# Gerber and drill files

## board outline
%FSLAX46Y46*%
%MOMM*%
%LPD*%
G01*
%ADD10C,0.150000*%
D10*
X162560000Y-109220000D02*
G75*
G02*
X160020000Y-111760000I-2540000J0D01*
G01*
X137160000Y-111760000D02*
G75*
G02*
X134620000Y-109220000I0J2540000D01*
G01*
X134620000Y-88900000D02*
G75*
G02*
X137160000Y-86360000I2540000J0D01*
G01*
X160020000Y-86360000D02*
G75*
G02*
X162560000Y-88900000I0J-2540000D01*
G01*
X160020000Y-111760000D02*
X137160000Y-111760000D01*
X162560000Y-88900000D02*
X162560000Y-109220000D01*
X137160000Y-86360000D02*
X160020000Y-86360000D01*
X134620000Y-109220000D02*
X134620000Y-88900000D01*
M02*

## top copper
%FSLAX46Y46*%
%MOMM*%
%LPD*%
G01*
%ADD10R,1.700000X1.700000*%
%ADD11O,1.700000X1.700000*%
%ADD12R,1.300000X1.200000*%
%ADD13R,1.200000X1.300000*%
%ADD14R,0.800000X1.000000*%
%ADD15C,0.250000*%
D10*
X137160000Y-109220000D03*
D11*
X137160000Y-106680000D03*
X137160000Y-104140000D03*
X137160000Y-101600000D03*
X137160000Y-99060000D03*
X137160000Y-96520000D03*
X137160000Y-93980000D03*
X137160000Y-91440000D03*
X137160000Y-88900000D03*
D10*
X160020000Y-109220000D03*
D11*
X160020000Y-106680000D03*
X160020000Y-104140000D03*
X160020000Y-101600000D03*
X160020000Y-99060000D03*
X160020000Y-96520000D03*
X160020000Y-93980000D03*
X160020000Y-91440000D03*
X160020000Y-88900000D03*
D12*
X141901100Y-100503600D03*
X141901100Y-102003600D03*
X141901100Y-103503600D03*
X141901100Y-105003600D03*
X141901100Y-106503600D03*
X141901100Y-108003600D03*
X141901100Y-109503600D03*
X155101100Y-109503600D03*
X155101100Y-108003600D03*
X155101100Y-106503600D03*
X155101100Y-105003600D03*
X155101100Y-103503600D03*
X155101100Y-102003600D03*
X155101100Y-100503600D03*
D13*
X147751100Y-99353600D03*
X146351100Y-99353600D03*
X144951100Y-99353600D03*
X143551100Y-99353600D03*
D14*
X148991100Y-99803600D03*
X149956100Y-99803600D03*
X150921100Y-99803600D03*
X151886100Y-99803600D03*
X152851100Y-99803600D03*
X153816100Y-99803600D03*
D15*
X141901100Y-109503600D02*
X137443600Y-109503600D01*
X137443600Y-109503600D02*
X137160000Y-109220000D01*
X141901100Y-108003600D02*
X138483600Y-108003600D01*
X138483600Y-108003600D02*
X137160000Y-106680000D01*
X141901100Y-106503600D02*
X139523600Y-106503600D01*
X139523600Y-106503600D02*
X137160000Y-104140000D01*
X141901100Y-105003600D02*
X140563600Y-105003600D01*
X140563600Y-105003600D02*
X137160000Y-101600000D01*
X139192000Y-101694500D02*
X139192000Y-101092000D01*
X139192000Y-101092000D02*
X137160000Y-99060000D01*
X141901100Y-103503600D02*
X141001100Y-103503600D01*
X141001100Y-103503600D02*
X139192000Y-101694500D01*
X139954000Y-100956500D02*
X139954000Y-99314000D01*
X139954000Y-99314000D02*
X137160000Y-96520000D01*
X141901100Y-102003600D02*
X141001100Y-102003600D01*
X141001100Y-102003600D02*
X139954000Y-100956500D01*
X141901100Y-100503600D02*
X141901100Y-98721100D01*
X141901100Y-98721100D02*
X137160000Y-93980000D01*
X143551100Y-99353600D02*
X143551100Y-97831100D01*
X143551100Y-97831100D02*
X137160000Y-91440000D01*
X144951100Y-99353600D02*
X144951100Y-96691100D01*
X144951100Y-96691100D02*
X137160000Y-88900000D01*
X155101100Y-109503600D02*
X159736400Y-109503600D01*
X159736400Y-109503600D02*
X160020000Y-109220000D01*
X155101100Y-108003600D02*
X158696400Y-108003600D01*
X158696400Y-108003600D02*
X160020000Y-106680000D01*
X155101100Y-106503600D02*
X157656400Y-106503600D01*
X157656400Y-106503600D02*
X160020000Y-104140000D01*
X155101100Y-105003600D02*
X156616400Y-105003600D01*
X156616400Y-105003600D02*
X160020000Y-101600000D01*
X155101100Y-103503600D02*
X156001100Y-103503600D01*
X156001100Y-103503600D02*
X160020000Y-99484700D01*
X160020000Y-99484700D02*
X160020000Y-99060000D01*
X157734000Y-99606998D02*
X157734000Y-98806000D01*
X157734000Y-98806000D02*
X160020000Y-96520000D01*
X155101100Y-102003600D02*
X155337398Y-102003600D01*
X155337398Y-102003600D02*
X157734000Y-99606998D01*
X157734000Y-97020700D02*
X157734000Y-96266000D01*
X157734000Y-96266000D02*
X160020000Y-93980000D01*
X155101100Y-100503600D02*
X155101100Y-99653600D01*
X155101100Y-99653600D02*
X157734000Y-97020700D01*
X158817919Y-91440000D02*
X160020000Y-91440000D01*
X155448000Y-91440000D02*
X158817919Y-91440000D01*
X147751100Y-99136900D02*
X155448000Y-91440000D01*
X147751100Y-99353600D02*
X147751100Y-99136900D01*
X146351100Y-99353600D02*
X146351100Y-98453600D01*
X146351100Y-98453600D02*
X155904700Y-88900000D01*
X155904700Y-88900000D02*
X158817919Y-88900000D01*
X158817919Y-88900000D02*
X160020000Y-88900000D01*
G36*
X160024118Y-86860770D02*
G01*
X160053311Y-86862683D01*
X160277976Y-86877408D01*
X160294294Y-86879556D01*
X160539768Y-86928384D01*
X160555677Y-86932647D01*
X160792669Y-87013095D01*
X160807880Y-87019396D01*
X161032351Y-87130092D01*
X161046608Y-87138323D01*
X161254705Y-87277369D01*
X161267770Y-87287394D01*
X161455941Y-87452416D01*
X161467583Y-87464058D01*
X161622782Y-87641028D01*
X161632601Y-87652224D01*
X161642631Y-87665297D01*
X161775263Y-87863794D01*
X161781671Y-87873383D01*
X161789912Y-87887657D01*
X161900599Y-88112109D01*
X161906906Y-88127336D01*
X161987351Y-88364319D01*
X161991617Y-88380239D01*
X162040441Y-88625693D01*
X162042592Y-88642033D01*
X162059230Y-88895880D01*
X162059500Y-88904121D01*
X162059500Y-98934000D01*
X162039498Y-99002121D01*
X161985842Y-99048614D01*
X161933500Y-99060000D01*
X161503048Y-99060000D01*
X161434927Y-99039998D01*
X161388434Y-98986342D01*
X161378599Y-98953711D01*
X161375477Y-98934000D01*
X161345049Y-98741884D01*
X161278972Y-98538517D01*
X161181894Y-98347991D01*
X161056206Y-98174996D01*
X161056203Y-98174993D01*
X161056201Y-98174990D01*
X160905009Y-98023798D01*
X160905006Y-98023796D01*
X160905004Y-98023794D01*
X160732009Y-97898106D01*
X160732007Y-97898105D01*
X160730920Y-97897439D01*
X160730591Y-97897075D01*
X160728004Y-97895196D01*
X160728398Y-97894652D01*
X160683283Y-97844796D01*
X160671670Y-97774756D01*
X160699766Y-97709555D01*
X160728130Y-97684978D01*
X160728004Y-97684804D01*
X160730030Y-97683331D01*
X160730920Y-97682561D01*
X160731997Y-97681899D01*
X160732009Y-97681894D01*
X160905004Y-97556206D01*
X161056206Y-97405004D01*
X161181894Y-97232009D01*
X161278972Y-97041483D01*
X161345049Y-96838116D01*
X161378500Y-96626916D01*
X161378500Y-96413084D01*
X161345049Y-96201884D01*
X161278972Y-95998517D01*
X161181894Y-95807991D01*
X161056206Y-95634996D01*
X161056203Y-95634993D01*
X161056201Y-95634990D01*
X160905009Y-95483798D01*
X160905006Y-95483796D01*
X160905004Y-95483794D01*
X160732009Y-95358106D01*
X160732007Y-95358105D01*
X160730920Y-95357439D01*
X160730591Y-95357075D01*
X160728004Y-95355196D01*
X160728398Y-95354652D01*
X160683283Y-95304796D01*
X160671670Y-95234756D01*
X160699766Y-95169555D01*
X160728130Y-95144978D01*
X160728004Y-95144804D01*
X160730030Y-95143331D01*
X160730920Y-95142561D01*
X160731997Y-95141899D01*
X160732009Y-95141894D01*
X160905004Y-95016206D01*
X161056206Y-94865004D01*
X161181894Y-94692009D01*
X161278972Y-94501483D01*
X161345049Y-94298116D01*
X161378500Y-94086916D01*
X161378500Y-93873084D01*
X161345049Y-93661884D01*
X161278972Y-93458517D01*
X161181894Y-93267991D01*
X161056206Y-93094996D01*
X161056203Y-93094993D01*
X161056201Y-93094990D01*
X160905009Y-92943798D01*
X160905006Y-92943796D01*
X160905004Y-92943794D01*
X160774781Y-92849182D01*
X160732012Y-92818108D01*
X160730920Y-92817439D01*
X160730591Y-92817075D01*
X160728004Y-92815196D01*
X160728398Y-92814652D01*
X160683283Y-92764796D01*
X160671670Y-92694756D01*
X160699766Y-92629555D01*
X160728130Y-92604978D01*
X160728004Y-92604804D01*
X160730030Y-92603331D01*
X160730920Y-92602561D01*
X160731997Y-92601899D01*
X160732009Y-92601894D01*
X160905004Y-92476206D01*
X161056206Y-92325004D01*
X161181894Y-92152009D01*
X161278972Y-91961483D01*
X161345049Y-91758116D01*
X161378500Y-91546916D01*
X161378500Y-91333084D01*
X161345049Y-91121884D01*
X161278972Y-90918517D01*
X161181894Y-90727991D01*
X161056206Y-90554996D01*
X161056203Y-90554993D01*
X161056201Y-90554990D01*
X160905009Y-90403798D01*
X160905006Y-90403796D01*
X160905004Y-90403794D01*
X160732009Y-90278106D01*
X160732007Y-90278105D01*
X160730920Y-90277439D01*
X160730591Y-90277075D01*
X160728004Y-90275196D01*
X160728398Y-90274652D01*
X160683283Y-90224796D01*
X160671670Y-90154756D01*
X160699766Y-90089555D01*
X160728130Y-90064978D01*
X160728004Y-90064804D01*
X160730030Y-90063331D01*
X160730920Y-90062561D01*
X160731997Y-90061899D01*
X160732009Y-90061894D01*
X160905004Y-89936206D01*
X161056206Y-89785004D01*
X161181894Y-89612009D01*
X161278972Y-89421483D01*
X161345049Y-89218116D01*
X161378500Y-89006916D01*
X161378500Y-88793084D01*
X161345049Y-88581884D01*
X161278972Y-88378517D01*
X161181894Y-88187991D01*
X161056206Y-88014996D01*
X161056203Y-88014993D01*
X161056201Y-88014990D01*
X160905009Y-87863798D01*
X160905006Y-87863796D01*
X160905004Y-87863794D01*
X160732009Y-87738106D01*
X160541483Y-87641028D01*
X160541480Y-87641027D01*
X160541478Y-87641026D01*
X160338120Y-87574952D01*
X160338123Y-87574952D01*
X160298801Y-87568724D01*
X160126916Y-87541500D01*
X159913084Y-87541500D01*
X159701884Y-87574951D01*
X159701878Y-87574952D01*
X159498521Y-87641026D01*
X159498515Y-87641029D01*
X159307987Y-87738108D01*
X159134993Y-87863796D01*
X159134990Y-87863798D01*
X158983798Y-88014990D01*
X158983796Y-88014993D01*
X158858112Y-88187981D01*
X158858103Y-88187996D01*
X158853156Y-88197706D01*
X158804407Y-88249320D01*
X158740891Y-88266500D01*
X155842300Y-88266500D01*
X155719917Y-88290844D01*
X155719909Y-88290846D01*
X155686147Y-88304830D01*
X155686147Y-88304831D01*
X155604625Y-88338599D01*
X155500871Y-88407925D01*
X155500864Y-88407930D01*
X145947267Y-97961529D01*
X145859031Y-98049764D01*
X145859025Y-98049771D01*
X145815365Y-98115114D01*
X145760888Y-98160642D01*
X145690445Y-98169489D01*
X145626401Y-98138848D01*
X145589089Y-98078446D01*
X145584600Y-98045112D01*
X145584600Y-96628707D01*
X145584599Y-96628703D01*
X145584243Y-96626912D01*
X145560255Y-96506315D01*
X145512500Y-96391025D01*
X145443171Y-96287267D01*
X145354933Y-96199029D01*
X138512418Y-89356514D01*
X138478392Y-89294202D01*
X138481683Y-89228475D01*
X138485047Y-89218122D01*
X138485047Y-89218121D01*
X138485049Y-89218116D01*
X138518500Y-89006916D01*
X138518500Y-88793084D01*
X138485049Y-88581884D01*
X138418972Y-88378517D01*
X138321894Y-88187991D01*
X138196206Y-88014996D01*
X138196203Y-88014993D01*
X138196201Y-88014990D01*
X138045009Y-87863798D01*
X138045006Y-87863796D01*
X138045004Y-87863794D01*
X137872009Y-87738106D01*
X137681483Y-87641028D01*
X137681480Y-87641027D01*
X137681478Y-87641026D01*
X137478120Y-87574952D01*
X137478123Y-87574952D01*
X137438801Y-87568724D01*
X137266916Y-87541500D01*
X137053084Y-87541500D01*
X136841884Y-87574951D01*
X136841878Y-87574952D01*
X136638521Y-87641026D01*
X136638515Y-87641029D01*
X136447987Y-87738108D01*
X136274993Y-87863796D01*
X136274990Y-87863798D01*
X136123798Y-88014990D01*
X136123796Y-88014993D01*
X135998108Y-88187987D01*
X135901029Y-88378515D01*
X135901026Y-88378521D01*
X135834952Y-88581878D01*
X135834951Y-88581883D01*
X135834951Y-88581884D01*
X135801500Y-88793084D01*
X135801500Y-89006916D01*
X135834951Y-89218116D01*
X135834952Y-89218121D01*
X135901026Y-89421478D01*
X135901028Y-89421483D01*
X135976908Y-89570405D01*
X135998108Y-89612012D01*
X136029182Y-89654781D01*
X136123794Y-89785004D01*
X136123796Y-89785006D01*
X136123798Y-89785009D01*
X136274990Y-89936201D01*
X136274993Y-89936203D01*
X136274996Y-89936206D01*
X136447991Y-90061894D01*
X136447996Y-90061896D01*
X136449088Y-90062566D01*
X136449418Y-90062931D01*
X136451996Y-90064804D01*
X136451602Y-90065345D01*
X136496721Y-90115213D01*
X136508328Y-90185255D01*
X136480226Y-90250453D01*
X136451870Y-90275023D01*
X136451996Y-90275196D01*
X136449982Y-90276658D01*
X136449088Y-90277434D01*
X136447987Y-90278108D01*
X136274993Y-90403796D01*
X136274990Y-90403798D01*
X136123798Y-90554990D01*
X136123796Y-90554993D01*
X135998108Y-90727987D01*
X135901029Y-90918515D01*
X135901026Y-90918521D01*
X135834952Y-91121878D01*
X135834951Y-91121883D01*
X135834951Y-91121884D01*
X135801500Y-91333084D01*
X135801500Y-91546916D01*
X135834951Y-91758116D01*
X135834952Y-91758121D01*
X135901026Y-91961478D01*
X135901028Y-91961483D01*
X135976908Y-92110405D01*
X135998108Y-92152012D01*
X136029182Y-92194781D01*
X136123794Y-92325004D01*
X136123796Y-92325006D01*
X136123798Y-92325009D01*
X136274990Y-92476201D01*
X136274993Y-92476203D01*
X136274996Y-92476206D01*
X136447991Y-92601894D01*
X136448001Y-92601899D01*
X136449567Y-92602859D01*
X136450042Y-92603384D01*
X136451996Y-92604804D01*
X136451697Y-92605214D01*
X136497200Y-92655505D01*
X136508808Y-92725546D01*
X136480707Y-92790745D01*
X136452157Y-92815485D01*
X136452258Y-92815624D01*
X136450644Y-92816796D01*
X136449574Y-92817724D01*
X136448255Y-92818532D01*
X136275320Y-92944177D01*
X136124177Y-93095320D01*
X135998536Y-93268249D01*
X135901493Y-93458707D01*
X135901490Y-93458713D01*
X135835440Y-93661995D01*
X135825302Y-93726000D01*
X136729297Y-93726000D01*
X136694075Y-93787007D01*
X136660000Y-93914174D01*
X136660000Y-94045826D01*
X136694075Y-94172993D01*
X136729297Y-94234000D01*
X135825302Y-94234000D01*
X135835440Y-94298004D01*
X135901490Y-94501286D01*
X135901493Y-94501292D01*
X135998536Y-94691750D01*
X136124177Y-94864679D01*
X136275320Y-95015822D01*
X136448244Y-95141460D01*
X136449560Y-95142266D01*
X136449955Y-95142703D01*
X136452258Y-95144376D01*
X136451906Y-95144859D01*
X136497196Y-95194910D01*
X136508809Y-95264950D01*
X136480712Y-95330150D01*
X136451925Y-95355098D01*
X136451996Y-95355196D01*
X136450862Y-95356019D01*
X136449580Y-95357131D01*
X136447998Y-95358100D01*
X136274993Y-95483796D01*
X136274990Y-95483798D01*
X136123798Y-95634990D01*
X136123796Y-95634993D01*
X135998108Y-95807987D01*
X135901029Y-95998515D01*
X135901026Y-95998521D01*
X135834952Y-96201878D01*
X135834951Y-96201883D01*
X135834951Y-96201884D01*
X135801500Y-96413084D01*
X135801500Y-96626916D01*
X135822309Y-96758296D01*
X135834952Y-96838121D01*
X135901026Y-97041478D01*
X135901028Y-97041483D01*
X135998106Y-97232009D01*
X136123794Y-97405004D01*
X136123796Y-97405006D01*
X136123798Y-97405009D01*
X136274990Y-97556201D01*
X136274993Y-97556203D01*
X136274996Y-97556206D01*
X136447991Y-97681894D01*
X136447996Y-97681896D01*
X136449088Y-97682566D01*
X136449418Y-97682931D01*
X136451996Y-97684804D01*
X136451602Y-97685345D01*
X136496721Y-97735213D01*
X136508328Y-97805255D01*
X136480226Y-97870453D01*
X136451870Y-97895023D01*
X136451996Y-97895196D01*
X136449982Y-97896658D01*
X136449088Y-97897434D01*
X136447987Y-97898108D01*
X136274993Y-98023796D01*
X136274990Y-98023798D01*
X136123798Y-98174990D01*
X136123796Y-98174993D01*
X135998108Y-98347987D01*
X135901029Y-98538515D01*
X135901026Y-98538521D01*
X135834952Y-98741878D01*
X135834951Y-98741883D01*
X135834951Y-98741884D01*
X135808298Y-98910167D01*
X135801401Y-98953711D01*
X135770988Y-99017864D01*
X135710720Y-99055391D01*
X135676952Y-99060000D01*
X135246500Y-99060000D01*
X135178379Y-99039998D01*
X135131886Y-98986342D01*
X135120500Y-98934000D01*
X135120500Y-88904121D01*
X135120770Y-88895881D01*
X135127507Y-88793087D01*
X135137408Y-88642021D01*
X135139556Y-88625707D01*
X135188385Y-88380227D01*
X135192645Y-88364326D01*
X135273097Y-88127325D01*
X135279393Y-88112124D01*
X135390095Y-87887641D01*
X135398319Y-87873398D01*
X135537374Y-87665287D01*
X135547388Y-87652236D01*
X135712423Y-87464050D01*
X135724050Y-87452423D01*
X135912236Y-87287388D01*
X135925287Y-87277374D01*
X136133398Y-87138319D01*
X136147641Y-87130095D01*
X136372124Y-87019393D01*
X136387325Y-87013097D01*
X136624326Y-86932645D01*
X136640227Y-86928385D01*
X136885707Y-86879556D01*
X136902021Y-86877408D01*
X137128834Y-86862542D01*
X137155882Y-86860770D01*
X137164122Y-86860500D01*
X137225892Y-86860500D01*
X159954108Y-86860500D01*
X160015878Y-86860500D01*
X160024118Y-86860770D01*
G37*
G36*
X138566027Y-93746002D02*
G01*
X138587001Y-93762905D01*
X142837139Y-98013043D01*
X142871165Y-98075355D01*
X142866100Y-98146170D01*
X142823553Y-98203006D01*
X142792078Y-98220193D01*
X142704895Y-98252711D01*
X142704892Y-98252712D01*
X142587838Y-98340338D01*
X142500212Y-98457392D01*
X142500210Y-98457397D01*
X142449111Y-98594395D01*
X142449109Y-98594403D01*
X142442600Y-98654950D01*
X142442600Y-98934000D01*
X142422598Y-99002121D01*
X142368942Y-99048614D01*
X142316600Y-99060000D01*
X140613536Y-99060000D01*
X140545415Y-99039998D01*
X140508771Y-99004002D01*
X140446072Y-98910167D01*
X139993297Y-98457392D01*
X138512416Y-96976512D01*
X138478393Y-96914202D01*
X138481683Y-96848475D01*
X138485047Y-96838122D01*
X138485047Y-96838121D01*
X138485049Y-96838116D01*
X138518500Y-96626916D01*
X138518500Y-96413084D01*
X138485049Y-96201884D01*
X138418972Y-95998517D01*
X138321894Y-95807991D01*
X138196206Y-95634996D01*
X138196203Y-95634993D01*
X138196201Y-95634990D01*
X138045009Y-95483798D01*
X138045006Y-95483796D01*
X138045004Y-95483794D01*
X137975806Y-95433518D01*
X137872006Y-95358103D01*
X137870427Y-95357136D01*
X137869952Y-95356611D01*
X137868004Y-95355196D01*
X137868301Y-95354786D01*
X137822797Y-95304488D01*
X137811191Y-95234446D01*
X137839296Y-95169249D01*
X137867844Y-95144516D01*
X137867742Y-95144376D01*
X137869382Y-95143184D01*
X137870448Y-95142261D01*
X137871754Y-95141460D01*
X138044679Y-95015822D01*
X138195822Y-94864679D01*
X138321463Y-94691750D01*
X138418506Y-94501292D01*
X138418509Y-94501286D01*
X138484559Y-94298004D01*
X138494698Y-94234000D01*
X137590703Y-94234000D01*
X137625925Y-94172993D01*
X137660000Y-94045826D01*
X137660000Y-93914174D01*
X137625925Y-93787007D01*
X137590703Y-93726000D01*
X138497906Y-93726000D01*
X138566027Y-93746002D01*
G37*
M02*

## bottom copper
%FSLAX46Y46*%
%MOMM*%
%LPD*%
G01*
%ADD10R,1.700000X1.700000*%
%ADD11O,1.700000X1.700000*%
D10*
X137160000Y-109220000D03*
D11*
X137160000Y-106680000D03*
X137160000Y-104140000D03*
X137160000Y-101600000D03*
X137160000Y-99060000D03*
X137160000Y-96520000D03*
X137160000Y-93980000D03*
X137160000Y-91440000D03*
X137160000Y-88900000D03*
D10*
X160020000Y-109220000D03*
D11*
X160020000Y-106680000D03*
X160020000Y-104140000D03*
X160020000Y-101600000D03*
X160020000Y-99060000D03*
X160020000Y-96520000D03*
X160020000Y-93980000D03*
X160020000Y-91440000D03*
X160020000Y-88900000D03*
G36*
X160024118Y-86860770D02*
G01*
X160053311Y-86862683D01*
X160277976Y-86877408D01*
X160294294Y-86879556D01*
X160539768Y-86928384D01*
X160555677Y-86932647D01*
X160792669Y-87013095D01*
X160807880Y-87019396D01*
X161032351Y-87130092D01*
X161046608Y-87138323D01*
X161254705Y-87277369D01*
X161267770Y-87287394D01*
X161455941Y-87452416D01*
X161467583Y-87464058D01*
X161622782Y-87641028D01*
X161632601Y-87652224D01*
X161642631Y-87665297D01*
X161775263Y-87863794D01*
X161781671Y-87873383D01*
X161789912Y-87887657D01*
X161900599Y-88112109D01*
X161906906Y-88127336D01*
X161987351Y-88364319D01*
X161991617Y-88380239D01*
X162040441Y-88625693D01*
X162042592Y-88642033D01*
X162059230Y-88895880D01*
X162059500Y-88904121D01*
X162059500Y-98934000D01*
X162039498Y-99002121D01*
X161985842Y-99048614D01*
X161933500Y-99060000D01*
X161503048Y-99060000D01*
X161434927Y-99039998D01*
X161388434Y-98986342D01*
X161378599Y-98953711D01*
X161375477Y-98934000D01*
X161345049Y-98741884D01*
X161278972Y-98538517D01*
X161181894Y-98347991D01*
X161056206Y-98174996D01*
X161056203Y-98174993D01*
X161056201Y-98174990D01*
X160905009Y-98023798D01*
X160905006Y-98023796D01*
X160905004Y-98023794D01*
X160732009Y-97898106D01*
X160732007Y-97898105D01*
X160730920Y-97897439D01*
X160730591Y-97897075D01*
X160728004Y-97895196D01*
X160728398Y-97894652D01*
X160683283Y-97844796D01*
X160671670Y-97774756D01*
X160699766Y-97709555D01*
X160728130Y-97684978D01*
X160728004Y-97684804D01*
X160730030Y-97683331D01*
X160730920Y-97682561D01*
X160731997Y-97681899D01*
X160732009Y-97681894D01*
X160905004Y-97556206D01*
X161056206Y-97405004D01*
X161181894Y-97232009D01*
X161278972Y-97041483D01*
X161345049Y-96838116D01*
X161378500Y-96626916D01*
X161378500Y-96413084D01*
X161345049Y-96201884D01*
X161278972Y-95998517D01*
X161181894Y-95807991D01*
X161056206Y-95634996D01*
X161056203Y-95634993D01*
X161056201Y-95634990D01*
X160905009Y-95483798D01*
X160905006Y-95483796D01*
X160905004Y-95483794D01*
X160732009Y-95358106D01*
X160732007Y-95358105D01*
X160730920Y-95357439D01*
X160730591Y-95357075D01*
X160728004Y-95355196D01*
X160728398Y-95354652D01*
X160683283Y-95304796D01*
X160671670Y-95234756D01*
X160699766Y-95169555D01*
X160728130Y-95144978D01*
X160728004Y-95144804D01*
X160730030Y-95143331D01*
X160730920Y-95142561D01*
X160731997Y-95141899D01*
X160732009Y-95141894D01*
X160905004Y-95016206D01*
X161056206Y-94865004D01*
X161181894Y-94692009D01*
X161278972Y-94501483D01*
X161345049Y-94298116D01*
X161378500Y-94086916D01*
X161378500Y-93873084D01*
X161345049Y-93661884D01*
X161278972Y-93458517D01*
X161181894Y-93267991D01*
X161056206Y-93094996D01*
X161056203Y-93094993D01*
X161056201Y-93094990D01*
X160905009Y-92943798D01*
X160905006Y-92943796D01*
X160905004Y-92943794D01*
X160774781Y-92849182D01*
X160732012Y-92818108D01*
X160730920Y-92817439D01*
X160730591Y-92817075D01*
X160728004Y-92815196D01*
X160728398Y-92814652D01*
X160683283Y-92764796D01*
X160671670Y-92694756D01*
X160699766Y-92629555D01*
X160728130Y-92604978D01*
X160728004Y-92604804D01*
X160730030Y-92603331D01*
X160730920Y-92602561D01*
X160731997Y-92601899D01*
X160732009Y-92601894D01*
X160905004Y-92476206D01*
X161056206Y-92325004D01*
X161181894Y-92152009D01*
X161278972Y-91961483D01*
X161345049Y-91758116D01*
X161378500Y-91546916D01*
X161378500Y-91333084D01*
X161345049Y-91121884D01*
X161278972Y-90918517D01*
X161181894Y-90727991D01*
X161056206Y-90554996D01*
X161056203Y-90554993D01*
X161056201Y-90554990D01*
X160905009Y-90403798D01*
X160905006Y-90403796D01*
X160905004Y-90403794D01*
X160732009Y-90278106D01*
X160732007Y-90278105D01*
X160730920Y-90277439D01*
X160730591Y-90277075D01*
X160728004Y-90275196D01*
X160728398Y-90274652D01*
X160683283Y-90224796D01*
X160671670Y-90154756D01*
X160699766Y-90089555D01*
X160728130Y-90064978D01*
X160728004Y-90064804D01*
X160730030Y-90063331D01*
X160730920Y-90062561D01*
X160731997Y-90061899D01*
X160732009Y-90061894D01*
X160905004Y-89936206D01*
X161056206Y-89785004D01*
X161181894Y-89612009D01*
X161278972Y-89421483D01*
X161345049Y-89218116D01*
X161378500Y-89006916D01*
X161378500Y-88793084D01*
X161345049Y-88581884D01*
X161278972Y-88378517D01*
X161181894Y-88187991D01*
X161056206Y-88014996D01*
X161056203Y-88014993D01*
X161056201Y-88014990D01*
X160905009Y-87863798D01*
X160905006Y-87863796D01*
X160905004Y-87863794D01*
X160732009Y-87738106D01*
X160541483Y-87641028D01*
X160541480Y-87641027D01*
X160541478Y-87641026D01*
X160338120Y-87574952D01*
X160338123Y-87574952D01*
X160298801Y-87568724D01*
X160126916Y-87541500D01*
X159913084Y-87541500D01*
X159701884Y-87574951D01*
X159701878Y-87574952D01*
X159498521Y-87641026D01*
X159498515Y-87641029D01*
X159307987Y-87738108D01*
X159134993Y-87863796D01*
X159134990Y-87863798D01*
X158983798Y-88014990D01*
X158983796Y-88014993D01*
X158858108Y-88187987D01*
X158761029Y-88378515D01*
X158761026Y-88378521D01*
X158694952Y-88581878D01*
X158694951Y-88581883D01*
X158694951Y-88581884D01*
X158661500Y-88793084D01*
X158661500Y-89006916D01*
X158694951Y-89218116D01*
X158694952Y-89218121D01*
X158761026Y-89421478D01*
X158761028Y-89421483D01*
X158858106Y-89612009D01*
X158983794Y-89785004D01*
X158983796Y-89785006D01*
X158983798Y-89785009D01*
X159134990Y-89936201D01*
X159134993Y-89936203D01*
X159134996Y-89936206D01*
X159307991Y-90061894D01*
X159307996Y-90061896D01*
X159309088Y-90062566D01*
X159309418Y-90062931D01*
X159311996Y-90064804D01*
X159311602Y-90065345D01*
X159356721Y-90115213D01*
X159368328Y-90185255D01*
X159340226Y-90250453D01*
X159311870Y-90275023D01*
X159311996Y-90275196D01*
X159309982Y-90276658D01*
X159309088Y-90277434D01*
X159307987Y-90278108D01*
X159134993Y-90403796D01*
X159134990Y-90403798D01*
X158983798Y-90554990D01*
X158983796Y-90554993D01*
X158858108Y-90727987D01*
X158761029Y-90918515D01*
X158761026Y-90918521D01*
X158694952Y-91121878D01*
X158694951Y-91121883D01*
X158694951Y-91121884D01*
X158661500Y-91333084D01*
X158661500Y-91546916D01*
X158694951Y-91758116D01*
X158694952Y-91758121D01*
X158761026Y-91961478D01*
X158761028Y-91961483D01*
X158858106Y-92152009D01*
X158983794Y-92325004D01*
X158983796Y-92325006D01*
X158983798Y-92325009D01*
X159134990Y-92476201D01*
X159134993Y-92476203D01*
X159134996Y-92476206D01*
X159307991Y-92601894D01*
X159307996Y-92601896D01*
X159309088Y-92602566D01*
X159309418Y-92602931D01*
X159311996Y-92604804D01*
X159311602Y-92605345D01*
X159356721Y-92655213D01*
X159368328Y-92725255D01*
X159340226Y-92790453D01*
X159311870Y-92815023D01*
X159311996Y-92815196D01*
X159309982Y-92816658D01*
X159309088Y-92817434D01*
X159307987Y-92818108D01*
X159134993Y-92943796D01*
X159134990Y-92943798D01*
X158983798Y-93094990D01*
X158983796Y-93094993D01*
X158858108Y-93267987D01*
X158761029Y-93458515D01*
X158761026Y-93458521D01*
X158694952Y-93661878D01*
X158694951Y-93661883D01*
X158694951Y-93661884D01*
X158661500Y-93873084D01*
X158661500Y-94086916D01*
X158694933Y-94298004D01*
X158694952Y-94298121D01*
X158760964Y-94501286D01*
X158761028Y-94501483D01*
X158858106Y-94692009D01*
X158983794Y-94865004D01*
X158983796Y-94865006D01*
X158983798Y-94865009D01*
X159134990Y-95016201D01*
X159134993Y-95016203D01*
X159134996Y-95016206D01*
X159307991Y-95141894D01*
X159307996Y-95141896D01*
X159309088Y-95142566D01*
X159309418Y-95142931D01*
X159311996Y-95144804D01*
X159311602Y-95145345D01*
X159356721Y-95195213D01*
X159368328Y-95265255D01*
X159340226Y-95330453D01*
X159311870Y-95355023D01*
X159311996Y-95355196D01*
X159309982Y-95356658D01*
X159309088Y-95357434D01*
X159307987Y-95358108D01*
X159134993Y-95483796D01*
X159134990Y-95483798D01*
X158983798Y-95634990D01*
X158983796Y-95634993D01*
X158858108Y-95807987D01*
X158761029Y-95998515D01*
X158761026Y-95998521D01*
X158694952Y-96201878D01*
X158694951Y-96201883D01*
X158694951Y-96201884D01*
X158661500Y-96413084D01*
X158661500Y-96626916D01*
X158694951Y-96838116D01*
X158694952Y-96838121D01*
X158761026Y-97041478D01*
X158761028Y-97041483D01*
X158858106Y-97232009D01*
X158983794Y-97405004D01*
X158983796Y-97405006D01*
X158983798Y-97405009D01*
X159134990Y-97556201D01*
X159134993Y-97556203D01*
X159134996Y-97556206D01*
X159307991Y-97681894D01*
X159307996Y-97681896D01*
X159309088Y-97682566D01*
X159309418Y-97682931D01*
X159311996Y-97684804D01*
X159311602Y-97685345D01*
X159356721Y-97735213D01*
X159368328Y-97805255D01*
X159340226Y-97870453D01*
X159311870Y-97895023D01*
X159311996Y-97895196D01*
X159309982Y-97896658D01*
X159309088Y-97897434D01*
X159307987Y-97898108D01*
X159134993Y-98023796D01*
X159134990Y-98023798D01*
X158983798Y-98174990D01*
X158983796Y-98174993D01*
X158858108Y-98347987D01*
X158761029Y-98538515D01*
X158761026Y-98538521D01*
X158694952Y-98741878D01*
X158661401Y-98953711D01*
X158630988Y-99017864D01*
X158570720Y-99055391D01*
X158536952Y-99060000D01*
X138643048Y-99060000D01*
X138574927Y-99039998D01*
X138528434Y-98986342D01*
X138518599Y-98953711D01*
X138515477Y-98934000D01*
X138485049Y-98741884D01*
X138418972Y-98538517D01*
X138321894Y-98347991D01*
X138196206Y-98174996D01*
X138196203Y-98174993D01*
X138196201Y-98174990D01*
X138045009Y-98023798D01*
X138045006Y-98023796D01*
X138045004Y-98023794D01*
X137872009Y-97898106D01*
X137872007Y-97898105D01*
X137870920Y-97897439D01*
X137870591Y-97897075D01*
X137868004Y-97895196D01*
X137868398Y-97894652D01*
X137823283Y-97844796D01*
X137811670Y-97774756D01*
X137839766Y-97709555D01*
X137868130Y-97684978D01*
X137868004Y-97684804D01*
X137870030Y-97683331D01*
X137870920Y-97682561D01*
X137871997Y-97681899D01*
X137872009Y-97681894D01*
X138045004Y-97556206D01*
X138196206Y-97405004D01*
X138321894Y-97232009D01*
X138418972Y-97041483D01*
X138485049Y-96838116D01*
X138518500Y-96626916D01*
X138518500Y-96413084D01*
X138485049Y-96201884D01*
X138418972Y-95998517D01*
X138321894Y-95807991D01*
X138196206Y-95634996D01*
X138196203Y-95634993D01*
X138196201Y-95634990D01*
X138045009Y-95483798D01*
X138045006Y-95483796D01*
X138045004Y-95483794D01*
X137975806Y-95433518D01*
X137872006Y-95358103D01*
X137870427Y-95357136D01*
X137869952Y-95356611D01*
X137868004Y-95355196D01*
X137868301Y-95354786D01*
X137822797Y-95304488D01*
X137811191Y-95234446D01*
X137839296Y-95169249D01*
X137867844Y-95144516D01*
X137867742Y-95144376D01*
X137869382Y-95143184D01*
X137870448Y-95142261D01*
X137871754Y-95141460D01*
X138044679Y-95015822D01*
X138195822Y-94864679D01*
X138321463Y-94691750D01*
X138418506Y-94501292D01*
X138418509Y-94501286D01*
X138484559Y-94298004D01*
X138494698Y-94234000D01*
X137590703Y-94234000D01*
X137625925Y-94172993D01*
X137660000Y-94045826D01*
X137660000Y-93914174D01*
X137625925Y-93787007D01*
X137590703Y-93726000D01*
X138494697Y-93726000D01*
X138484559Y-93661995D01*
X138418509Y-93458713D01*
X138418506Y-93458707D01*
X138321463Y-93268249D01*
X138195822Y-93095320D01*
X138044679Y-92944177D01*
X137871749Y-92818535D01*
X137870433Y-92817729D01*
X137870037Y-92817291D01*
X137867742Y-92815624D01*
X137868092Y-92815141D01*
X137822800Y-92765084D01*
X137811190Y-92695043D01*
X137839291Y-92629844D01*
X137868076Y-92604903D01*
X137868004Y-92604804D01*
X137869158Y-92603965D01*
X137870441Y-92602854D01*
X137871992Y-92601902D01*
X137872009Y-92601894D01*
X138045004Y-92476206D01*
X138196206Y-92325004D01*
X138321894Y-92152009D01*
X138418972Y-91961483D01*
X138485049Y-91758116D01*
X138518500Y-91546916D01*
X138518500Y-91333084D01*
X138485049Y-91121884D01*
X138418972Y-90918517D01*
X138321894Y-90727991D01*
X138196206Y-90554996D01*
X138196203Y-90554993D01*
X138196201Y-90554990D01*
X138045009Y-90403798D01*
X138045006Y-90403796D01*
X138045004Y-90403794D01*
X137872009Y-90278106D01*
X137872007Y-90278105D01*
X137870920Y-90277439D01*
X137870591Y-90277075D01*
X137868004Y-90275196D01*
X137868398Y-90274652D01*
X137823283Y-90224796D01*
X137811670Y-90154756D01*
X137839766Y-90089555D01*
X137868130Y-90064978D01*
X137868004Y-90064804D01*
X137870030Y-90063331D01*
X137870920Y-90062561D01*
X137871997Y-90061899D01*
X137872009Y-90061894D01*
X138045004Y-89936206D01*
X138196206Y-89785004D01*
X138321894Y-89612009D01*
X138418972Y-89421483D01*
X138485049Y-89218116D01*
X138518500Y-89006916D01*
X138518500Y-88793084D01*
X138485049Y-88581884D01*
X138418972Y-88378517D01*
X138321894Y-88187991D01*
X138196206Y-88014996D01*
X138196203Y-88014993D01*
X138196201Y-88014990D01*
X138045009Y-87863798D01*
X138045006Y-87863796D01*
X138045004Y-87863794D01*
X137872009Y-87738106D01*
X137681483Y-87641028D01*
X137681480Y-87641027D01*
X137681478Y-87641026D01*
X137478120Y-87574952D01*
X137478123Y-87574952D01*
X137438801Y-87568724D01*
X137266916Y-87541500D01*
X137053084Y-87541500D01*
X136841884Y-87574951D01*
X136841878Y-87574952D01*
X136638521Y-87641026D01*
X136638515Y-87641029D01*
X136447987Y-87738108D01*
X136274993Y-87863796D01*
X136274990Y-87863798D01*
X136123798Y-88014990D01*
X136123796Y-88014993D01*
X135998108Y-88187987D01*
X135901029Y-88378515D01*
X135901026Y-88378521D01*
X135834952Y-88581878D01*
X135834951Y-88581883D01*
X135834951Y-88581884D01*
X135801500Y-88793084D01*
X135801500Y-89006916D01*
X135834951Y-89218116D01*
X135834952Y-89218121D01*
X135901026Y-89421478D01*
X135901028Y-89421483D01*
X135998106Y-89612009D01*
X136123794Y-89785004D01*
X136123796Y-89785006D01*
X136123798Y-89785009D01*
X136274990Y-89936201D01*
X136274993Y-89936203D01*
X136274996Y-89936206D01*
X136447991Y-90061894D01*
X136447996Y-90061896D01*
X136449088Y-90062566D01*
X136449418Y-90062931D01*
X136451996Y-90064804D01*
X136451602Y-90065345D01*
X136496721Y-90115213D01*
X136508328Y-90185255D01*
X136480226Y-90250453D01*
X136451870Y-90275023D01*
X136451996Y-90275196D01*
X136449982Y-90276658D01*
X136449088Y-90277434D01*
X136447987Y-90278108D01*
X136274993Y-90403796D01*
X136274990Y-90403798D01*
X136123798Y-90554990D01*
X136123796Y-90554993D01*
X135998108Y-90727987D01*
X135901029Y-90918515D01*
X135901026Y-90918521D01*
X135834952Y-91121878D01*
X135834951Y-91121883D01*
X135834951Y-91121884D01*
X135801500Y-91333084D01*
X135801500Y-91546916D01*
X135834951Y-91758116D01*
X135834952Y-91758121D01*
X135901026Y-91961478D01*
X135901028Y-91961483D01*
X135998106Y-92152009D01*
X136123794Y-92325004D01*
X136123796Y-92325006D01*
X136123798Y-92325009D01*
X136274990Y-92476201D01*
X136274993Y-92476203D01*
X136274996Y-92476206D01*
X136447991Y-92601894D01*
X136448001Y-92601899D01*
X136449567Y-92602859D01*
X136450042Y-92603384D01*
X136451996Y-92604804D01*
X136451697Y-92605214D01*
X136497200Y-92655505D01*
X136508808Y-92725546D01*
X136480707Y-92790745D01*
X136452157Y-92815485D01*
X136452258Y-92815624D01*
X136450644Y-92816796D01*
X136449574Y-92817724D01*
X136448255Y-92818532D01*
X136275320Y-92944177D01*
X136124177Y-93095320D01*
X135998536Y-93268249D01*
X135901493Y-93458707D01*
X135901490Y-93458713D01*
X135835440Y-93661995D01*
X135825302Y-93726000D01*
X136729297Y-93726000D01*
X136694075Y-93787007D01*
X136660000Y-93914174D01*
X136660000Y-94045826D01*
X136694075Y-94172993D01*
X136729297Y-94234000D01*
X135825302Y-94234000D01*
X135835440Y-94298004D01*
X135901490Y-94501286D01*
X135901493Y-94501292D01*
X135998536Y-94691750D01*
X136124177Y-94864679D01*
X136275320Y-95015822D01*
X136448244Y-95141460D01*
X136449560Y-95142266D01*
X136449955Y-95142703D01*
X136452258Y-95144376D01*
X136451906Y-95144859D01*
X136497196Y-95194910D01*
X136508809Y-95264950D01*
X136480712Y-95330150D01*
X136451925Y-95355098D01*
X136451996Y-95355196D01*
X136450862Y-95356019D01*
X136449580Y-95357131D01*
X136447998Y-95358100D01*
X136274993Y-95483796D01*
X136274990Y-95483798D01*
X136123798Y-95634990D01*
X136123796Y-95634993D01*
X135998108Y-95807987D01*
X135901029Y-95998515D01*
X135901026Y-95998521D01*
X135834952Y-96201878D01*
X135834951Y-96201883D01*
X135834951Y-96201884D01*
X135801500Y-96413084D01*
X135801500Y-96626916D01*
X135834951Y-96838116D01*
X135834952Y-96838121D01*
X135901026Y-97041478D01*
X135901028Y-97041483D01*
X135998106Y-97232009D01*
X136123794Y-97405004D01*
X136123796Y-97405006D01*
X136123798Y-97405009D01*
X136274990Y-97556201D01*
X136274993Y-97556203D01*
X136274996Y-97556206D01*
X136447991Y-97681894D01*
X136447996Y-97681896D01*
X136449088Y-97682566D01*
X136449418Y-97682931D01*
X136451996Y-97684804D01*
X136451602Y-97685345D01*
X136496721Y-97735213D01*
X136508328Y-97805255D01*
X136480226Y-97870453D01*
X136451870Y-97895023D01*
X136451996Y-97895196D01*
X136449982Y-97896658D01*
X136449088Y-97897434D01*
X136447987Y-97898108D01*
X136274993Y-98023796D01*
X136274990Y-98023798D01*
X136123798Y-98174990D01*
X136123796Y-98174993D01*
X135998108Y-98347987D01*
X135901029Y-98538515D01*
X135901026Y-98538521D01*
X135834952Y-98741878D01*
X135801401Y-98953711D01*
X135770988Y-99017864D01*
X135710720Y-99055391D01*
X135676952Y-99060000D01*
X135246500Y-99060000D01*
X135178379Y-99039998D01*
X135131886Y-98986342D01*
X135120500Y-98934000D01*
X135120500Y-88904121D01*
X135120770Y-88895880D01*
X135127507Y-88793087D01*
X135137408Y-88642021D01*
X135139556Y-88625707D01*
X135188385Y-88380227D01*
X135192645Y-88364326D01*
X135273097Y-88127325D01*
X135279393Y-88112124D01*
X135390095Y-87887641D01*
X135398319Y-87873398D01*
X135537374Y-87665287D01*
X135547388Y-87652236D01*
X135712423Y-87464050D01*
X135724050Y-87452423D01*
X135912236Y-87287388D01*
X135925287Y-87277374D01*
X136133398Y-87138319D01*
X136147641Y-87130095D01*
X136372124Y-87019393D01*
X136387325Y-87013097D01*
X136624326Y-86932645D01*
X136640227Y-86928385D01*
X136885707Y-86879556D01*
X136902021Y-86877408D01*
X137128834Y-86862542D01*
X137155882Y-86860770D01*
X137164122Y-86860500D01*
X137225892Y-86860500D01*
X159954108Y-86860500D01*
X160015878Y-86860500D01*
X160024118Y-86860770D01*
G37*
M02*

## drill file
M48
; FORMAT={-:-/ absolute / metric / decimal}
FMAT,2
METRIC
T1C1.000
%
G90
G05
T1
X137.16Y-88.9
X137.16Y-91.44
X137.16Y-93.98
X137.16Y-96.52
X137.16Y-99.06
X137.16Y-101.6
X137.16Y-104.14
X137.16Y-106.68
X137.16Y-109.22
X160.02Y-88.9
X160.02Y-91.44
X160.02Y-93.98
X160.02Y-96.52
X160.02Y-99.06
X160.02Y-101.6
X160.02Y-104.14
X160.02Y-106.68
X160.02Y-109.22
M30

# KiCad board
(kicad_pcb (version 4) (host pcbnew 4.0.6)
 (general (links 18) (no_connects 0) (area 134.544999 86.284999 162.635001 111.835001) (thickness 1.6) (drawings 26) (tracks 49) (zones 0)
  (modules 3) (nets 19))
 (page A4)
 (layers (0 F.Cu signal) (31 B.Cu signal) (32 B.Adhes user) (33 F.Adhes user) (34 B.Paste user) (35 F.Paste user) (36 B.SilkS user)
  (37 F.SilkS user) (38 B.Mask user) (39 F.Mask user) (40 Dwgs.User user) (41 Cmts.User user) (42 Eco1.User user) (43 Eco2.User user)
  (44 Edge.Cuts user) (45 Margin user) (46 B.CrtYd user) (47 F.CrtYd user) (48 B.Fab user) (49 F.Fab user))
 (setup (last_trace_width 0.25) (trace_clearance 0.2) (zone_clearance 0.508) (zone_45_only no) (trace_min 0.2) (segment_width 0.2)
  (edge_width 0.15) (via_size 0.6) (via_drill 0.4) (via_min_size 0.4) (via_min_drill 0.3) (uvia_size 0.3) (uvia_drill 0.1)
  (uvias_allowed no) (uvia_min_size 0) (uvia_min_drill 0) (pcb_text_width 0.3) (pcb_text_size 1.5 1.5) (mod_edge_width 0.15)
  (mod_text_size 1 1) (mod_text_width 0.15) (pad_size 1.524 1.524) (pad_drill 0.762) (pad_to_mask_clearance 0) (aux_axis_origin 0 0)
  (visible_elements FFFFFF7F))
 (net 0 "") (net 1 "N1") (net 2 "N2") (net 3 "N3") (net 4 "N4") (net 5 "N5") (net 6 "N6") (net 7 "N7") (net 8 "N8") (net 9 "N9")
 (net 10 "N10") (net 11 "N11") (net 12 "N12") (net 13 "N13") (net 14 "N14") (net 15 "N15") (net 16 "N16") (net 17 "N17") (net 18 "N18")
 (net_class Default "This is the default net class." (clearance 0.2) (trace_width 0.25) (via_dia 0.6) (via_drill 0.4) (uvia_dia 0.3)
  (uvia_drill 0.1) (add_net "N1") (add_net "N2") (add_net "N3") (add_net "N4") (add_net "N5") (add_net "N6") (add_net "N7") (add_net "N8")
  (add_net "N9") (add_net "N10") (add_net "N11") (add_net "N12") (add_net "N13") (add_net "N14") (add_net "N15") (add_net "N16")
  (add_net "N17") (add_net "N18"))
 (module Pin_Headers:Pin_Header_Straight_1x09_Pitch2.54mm (layer F.Cu) (at 137.16 109.22 180)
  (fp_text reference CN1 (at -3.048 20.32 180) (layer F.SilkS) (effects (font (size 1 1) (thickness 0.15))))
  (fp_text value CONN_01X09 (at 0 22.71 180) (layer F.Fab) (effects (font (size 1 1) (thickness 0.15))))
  (pad 1 thru_hole rect (at 0 0 180) (size 1.7 1.7) (drill 1) (layers *.Cu *.Mask) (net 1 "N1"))
  (pad 2 thru_hole oval (at 0 2.54 180) (size 1.7 1.7) (drill 1) (layers *.Cu *.Mask) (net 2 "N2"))
  (pad 3 thru_hole oval (at 0 5.08 180) (size 1.7 1.7) (drill 1) (layers *.Cu *.Mask) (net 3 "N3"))
  (pad 4 thru_hole oval (at 0 7.62 180) (size 1.7 1.7) (drill 1) (layers *.Cu *.Mask) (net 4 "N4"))
  (pad 5 thru_hole oval (at 0 10.16 180) (size 1.7 1.7) (drill 1) (layers *.Cu *.Mask) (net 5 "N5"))
  (pad 6 thru_hole oval (at 0 12.7 180) (size 1.7 1.7) (drill 1) (layers *.Cu *.Mask) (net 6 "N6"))
  (pad 7 thru_hole oval (at 0 15.24 180) (size 1.7 1.7) (drill 1) (layers *.Cu *.Mask) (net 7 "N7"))
  (pad 8 thru_hole oval (at 0 17.78 180) (size 1.7 1.7) (drill 1) (layers *.Cu *.Mask) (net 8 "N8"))
  (pad 9 thru_hole oval (at 0 20.32 180) (size 1.7 1.7) (drill 1) (layers *.Cu *.Mask) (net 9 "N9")))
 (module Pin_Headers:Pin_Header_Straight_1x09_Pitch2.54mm (layer F.Cu) (at 160.02 109.22 180)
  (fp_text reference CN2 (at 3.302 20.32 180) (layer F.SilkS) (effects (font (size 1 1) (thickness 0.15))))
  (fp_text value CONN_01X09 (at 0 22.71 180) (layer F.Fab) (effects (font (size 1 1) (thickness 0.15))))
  (pad 1 thru_hole rect (at 0 0 180) (size 1.7 1.7) (drill 1) (layers *.Cu *.Mask) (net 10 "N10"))
  (pad 2 thru_hole oval (at 0 2.54 180) (size 1.7 1.7) (drill 1) (layers *.Cu *.Mask) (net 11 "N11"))
  (pad 3 thru_hole oval (at 0 5.08 180) (size 1.7 1.7) (drill 1) (layers *.Cu *.Mask) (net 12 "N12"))
  (pad 4 thru_hole oval (at 0 7.62 180) (size 1.7 1.7) (drill 1) (layers *.Cu *.Mask) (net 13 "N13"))
  (pad 5 thru_hole oval (at 0 10.16 180) (size 1.7 1.7) (drill 1) (layers *.Cu *.Mask) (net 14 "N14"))
  (pad 6 thru_hole oval (at 0 12.7 180) (size 1.7 1.7) (drill 1) (layers *.Cu *.Mask) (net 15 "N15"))
  (pad 7 thru_hole oval (at 0 15.24 180) (size 1.7 1.7) (drill 1) (layers *.Cu *.Mask) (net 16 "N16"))
  (pad 8 thru_hole oval (at 0 17.78 180) (size 1.7 1.7) (drill 1) (layers *.Cu *.Mask) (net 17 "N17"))
  (pad 9 thru_hole oval (at 0 20.32 180) (size 1.7 1.7) (drill 1) (layers *.Cu *.Mask) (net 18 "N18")))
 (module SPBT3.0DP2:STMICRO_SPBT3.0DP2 (layer F.Cu) (at 148.5011 105.0036)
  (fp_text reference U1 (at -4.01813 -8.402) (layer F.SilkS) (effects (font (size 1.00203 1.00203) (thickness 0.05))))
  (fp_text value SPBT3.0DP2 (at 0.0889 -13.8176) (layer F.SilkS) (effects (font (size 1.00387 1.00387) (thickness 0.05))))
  (pad 1 smd rect (at -6.6 -4.5 270) (size 1.2 1.3) (layers F.Cu F.Paste F.Mask) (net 7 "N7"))
  (pad 2 smd rect (at -6.6 -3 270) (size 1.2 1.3) (layers F.Cu F.Paste F.Mask) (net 6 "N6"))
  (pad 3 smd rect (at -6.6 -1.5 270) (size 1.2 1.3) (layers F.Cu F.Paste F.Mask) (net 5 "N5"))
  (pad 4 smd rect (at -6.6 0 270) (size 1.2 1.3) (layers F.Cu F.Paste F.Mask) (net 4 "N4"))
  (pad 5 smd rect (at -6.6 1.5 270) (size 1.2 1.3) (layers F.Cu F.Paste F.Mask) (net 3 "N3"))
  (pad 6 smd rect (at -6.6 3 270) (size 1.2 1.3) (layers F.Cu F.Paste F.Mask) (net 2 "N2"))
  (pad 7 smd rect (at -6.6 4.5 270) (size 1.2 1.3) (layers F.Cu F.Paste F.Mask) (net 1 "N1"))
  (pad 8 smd rect (at 6.6 4.5 270) (size 1.2 1.3) (layers F.Cu F.Paste F.Mask) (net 10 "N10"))
  (pad 9 smd rect (at 6.6 3 270) (size 1.2 1.3) (layers F.Cu F.Paste F.Mask) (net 11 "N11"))
  (pad 10 smd rect (at 6.6 1.5 270) (size 1.2 1.3) (layers F.Cu F.Paste F.Mask) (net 12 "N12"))
  (pad 11 smd rect (at 6.6 0 270) (size 1.2 1.3) (layers F.Cu F.Paste F.Mask) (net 13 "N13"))
  (pad 12 smd rect (at 6.6 -1.5 270) (size 1.2 1.3) (layers F.Cu F.Paste F.Mask) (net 14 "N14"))
  (pad 13 smd rect (at 6.6 -3 270) (size 1.2 1.3) (layers F.Cu F.Paste F.Mask) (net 15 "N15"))
  (pad 14 smd rect (at 6.6 -4.5 270) (size 1.2 1.3) (layers F.Cu F.Paste F.Mask) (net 16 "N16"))
  (pad 15 smd rect (at -0.75 -5.65) (size 1.2 1.3) (layers F.Cu F.Paste F.Mask) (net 17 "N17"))
  (pad 16 smd rect (at -2.15 -5.65) (size 1.2 1.3) (layers F.Cu F.Paste F.Mask) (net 18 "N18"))
  (pad 17 smd rect (at -3.55 -5.65) (size 1.2 1.3) (layers F.Cu F.Paste F.Mask) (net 9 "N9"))
  (pad 18 smd rect (at -4.95 -5.65) (size 1.2 1.3) (layers F.Cu F.Paste F.Mask) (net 8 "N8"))
  (pad P$6 smd rect (at 0.49 -5.2) (size 0.8 1) (layers F.Cu F.Paste F.Mask))
  (pad P$5 smd rect (at 1.455 -5.2) (size 0.8 1) (layers F.Cu F.Paste F.Mask))
  (pad P$4 smd rect (at 2.42 -5.2) (size 0.8 1) (layers F.Cu F.Paste F.Mask))
  (pad P$3 smd rect (at 3.385 -5.2) (size 0.8 1) (layers F.Cu F.Paste F.Mask))
  (pad P$2 smd rect (at 4.35 -5.2) (size 0.8 1) (layers F.Cu F.Paste F.Mask))
  (pad P$1 smd rect (at 5.315 -5.2) (size 0.8 1) (layers F.Cu F.Paste F.Mask)))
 (gr_arc (start 160.02 109.22) (end 162.56 109.22) (angle 90) (layer Edge.Cuts) (width 0.15))
 (gr_arc (start 137.16 109.22) (end 137.16 111.76) (angle 90) (layer Edge.Cuts) (width 0.15))
 (gr_arc (start 137.16 88.9) (end 134.62 88.9) (angle 90) (layer Edge.Cuts) (width 0.15))
 (gr_arc (start 160.02 88.9) (end 160.02 86.36) (angle 90) (layer Edge.Cuts) (width 0.15))
 (gr_line (start 160.02 111.76) (end 137.16 111.76) (layer Edge.Cuts) (width 0.15))
 (gr_line (start 162.56 88.9) (end 162.56 109.22) (layer Edge.Cuts) (width 0.15))
 (gr_line (start 137.16 86.36) (end 160.02 86.36) (layer Edge.Cuts) (width 0.15))
 (gr_line (start 134.62 109.22) (end 134.62 88.9) (layer Edge.Cuts) (width 0.15))
 (segment (start 141.9011 109.5036) (end 137.4436 109.5036) (width 0.25) (layer F.Cu) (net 1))
 (segment (start 137.4436 109.5036) (end 137.16 109.22) (width 0.25) (layer F.Cu) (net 1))
 (segment (start 141.9011 108.0036) (end 138.4836 108.0036) (width 0.25) (layer F.Cu) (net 2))
 (segment (start 138.4836 108.0036) (end 137.16 106.68) (width 0.25) (layer F.Cu) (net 2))
 (segment (start 141.9011 106.5036) (end 139.5236 106.5036) (width 0.25) (layer F.Cu) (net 3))
 (segment (start 139.5236 106.5036) (end 137.16 104.14) (width 0.25) (layer F.Cu) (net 3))
 (segment (start 141.9011 105.0036) (end 140.5636 105.0036) (width 0.25) (layer F.Cu) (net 4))
 (segment (start 140.5636 105.0036) (end 137.16 101.6) (width 0.25) (layer F.Cu) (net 4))
 (segment (start 139.192 101.6945) (end 139.192 101.092) (width 0.25) (layer F.Cu) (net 5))
 (segment (start 139.192 101.092) (end 137.16 99.06) (width 0.25) (layer F.Cu) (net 5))
 (segment (start 141.9011 103.5036) (end 141.0011 103.5036) (width 0.25) (layer F.Cu) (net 5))
 (segment (start 141.0011 103.5036) (end 139.192 101.6945) (width 0.25) (layer F.Cu) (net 5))
 (segment (start 139.954 100.9565) (end 139.954 99.314) (width 0.25) (layer F.Cu) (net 6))
 (segment (start 139.954 99.314) (end 137.16 96.52) (width 0.25) (layer F.Cu) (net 6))
 (segment (start 141.9011 102.0036) (end 141.0011 102.0036) (width 0.25) (layer F.Cu) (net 6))
 (segment (start 141.0011 102.0036) (end 139.954 100.9565) (width 0.25) (layer F.Cu) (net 6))
 (segment (start 141.9011 100.5036) (end 141.9011 98.7211) (width 0.25) (layer F.Cu) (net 7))
 (segment (start 141.9011 98.7211) (end 137.16 93.98) (width 0.25) (layer F.Cu) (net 7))
 (segment (start 143.5511 99.3536) (end 143.5511 97.8311) (width 0.25) (layer F.Cu) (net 8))
 (segment (start 143.5511 97.8311) (end 137.16 91.44) (width 0.25) (layer F.Cu) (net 8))
 (segment (start 144.9511 99.3536) (end 144.9511 96.6911) (width 0.25) (layer F.Cu) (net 9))
 (segment (start 144.9511 96.6911) (end 137.16 88.9) (width 0.25) (layer F.Cu) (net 9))
 (segment (start 155.1011 109.5036) (end 159.7364 109.5036) (width 0.25) (layer F.Cu) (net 10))
 (segment (start 159.7364 109.5036) (end 160.02 109.22) (width 0.25) (layer F.Cu) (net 10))
 (segment (start 155.1011 108.0036) (end 158.6964 108.0036) (width 0.25) (layer F.Cu) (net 11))
 (segment (start 158.6964 108.0036) (end 160.02 106.68) (width 0.25) (layer F.Cu) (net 11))
 (segment (start 155.1011 106.5036) (end 157.6564 106.5036) (width 0.25) (layer F.Cu) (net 12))
 (segment (start 157.6564 106.5036) (end 160.02 104.14) (width 0.25) (layer F.Cu) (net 12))
 (segment (start 155.1011 105.0036) (end 156.6164 105.0036) (width 0.25) (layer F.Cu) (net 13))
 (segment (start 156.6164 105.0036) (end 160.02 101.6) (width 0.25) (layer F.Cu) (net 13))
 (segment (start 155.1011 103.5036) (end 156.0011 103.5036) (width 0.25) (layer F.Cu) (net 14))
 (segment (start 156.0011 103.5036) (end 160.02 99.4847) (width 0.25) (layer F.Cu) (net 14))
 (segment (start 160.02 99.4847) (end 160.02 99.06) (width 0.25) (layer F.Cu) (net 14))
 (segment (start 157.734 99.606998) (end 157.734 98.806) (width 0.25) (layer F.Cu) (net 15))
 (segment (start 157.734 98.806) (end 160.02 96.52) (width 0.25) (layer F.Cu) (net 15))
 (segment (start 155.1011 102.0036) (end 155.337398 102.0036) (width 0.25) (layer F.Cu) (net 15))
 (segment (start 155.337398 102.0036) (end 157.734 99.606998) (width 0.25) (layer F.Cu) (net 15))
 (segment (start 157.734 97.0207) (end 157.734 96.266) (width 0.25) (layer F.Cu) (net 16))
 (segment (start 157.734 96.266) (end 160.02 93.98) (width 0.25) (layer F.Cu) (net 16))
 (segment (start 155.1011 100.5036) (end 155.1011 99.6536) (width 0.25) (layer F.Cu) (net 16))
 (segment (start 155.1011 99.6536) (end 157.734 97.0207) (width 0.25) (layer F.Cu) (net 16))
 (segment (start 158.817919 91.44) (end 160.02 91.44) (width 0.25) (layer F.Cu) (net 17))
 (segment (start 155.448 91.44) (end 158.817919 91.44) (width 0.25) (layer F.Cu) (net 17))
 (segment (start 147.7511 99.1369) (end 155.448 91.44) (width 0.25) (layer F.Cu) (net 17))
 (segment (start 147.7511 99.3536) (end 147.7511 99.1369) (width 0.25) (layer F.Cu) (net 17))
 (segment (start 146.3511 99.3536) (end 146.3511 98.4536) (width 0.25) (layer F.Cu) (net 18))
 (segment (start 146.3511 98.4536) (end 155.9047 88.9) (width 0.25) (layer F.Cu) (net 18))
 (segment (start 155.9047 88.9) (end 158.817919 88.9) (width 0.25) (layer F.Cu) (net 18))
 (segment (start 158.817919 88.9) (end 160.02 88.9) (width 0.25) (layer F.Cu) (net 18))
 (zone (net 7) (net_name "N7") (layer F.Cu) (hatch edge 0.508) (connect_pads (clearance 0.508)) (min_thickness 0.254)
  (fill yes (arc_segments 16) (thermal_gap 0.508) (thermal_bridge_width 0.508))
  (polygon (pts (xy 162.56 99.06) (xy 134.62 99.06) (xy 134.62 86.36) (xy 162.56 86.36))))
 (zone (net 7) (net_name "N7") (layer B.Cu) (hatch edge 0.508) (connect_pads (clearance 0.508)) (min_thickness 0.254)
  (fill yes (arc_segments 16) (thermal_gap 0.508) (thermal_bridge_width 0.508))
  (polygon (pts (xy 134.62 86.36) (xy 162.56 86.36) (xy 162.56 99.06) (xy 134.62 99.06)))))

